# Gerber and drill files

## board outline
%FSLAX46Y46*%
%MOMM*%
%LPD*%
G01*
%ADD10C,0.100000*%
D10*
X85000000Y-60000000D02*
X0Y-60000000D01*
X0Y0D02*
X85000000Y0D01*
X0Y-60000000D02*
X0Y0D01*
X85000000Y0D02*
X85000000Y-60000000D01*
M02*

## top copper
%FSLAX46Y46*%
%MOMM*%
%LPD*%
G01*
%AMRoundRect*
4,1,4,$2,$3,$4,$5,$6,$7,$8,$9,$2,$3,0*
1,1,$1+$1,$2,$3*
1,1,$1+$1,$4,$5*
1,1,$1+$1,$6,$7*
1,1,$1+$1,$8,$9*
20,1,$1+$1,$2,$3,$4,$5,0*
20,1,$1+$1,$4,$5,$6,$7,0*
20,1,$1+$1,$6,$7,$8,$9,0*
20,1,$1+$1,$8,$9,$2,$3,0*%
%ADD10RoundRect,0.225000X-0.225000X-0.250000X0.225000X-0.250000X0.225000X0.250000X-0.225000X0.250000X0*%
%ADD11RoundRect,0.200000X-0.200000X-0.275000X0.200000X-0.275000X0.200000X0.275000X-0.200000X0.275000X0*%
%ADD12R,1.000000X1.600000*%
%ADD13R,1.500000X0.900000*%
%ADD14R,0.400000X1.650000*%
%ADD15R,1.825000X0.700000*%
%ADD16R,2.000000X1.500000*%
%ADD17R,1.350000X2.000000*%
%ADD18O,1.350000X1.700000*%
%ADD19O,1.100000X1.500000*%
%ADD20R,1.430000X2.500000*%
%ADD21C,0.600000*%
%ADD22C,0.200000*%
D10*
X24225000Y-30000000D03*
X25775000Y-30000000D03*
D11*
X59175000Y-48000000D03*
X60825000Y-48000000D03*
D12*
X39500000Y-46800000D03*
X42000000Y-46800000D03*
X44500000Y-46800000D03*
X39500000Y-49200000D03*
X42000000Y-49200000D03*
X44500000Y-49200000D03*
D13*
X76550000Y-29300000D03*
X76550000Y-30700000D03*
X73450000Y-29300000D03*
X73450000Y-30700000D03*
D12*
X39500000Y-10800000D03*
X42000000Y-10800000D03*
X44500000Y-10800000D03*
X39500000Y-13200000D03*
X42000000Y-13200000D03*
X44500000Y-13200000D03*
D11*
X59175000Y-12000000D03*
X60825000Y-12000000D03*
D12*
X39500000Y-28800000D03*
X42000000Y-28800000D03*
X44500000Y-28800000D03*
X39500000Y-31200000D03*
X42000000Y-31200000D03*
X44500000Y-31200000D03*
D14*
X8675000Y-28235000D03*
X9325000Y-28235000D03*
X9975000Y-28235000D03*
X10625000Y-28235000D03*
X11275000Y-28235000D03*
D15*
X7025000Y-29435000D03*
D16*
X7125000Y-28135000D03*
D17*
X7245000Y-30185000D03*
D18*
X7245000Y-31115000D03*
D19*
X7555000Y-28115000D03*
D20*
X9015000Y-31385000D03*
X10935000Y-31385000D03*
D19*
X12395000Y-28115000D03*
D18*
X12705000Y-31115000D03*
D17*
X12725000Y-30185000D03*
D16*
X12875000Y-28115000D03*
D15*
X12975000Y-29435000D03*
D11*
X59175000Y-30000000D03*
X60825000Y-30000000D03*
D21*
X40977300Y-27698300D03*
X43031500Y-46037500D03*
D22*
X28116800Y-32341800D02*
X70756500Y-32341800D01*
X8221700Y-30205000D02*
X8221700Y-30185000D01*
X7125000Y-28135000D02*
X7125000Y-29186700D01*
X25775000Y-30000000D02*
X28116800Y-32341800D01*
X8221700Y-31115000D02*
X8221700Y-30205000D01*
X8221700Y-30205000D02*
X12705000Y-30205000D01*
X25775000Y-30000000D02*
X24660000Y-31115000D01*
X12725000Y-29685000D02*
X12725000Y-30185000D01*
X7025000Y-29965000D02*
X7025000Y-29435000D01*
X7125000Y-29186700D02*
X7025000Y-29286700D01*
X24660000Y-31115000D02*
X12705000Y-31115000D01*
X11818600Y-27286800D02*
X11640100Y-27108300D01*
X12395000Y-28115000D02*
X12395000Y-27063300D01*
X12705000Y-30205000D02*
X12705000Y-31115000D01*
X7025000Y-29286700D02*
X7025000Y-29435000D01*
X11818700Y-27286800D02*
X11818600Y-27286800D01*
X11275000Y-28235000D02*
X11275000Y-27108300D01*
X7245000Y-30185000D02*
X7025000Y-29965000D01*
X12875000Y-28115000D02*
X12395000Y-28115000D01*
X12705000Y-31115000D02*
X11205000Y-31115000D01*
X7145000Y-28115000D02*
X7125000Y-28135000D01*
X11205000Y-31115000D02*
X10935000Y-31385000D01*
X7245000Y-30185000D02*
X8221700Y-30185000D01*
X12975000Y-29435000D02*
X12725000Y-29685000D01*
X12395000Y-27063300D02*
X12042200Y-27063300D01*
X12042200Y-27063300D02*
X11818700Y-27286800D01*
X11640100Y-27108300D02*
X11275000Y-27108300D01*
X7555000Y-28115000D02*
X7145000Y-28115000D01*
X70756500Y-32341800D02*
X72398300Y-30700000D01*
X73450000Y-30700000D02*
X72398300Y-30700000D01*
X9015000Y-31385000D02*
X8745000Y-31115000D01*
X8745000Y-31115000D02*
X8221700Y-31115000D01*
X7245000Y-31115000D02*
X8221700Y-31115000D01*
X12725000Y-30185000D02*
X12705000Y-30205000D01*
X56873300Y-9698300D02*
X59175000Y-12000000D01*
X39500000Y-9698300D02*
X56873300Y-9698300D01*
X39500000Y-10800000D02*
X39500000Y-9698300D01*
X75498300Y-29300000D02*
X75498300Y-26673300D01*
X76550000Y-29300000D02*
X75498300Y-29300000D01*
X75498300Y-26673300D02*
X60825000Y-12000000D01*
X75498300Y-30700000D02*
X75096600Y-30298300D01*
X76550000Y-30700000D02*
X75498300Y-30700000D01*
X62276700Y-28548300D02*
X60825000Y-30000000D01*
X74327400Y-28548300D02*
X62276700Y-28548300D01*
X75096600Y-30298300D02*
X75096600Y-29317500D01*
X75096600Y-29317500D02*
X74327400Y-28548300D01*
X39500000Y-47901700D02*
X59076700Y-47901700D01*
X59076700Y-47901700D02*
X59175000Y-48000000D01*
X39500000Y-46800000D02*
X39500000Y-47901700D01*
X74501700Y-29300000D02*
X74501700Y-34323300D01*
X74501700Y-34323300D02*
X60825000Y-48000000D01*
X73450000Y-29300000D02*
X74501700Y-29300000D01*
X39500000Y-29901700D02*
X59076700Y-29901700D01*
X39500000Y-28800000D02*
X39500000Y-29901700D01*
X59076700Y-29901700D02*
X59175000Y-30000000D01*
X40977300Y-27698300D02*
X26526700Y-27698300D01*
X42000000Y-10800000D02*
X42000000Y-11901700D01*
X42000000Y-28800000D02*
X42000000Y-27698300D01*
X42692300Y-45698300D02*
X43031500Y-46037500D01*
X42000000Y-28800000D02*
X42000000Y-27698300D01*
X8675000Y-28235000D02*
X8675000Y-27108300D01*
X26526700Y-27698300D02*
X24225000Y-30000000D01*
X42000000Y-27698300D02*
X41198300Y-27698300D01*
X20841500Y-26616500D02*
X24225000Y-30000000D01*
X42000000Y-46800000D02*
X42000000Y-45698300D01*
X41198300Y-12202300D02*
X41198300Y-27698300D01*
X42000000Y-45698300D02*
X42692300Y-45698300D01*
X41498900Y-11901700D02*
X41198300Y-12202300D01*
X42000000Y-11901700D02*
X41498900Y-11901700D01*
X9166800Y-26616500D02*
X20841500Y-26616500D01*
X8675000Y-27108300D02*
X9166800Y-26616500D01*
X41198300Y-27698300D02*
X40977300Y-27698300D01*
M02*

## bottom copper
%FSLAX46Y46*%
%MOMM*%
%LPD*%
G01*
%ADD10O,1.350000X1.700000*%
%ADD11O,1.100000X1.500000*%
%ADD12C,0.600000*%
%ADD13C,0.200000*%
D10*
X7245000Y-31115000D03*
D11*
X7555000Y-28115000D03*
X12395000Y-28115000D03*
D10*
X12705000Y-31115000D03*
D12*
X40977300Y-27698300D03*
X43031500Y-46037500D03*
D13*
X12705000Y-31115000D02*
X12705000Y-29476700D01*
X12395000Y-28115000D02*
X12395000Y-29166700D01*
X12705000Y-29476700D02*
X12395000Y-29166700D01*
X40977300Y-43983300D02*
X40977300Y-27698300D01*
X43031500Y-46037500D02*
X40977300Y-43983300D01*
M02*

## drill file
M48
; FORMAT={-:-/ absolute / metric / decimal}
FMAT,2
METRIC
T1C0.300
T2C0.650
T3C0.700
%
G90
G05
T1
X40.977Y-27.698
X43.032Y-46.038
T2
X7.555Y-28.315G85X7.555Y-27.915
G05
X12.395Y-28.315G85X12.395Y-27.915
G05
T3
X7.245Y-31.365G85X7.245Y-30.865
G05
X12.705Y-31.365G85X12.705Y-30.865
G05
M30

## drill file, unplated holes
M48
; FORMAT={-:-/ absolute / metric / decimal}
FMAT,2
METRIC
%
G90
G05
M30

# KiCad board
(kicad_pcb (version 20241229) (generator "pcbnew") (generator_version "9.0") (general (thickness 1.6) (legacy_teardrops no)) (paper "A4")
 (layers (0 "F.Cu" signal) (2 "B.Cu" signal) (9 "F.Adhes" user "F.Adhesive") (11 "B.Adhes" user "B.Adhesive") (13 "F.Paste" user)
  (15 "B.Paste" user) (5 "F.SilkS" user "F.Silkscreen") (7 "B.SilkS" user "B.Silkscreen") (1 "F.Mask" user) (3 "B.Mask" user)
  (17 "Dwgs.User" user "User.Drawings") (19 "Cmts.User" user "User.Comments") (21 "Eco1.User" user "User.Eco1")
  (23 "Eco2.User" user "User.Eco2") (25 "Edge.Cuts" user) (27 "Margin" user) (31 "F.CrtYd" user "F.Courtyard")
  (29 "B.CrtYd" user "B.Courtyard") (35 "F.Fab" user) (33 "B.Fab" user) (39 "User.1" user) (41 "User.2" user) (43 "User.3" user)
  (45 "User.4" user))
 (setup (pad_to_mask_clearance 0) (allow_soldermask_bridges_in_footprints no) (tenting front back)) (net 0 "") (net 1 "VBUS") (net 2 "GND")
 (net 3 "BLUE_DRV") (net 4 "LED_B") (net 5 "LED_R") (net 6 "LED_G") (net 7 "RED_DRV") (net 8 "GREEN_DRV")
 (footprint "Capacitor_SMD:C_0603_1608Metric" (layer "F.Cu") (at 25 30)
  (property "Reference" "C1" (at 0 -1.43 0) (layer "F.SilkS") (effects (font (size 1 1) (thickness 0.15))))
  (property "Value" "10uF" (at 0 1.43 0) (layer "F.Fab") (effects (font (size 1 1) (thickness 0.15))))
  (pad "1" smd roundrect (at -0.775 0) (size 0.9 0.95) (layers "F.Cu" "F.Mask" "F.Paste") (roundrect_rratio 0.25) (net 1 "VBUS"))
  (pad "2" smd roundrect (at 0.775 0) (size 0.9 0.95) (layers "F.Cu" "F.Mask" "F.Paste") (roundrect_rratio 0.25) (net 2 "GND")))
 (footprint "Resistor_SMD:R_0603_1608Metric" (layer "F.Cu") (at 60 48)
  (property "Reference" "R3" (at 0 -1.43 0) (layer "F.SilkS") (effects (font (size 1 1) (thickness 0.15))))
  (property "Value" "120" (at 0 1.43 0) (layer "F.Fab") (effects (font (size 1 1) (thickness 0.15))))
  (pad "1" smd roundrect (at -0.825 0) (size 0.8 0.95) (layers "F.Cu" "F.Mask" "F.Paste") (roundrect_rratio 0.25) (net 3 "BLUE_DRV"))
  (pad "2" smd roundrect (at 0.825 0) (size 0.8 0.95) (layers "F.Cu" "F.Mask" "F.Paste") (roundrect_rratio 0.25) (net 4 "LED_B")))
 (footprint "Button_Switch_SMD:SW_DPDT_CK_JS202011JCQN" (layer "F.Cu") (at 42 48)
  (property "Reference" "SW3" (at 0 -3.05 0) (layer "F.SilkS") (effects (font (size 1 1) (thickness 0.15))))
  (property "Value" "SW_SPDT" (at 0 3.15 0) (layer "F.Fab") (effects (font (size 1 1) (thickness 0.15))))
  (pad "1" smd rect (at -2.5 -1.2) (size 1 1.6) (layers "F.Cu" "F.Mask" "F.Paste") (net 3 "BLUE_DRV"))
  (pad "2" smd rect (at 0 -1.2) (size 1 1.6) (layers "F.Cu" "F.Mask" "F.Paste") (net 1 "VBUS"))
  (pad "3" smd rect (at 2.5 -1.2) (size 1 1.6) (layers "F.Cu" "F.Mask" "F.Paste"))
  (pad "4" smd rect (at -2.5 1.2) (size 1 1.6) (layers "F.Cu" "F.Mask" "F.Paste"))
  (pad "5" smd rect (at 0 1.2) (size 1 1.6) (layers "F.Cu" "F.Mask" "F.Paste"))
  (pad "6" smd rect (at 2.5 1.2) (size 1 1.6) (layers "F.Cu" "F.Mask" "F.Paste")))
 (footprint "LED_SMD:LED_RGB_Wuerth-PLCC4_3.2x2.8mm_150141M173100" (layer "F.Cu") (at 75 30)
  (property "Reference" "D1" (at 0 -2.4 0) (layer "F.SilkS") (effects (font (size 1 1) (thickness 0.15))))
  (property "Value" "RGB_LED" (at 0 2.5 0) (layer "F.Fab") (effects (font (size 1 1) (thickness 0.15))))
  (pad "1" smd rect (at 1.55 -0.7) (size 1.5 0.9) (layers "F.Cu" "F.Mask" "F.Paste") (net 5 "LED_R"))
  (pad "2" smd rect (at 1.55 0.7) (size 1.5 0.9) (layers "F.Cu" "F.Mask" "F.Paste") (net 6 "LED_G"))
  (pad "3" smd rect (at -1.55 -0.7) (size 1.5 0.9) (layers "F.Cu" "F.Mask" "F.Paste") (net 4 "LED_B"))
  (pad "4" smd rect (at -1.55 0.7) (size 1.5 0.9) (layers "F.Cu" "F.Mask" "F.Paste") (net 2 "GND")))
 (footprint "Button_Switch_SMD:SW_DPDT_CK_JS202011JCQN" (layer "F.Cu") (at 42 12)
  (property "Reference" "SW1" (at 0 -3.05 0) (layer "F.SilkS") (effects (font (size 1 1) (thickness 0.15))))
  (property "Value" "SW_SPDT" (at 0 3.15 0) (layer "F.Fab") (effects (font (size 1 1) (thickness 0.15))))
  (pad "1" smd rect (at -2.5 -1.2) (size 1 1.6) (layers "F.Cu" "F.Mask" "F.Paste") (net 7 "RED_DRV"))
  (pad "2" smd rect (at 0 -1.2) (size 1 1.6) (layers "F.Cu" "F.Mask" "F.Paste") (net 1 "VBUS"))
  (pad "3" smd rect (at 2.5 -1.2) (size 1 1.6) (layers "F.Cu" "F.Mask" "F.Paste"))
  (pad "4" smd rect (at -2.5 1.2) (size 1 1.6) (layers "F.Cu" "F.Mask" "F.Paste"))
  (pad "5" smd rect (at 0 1.2) (size 1 1.6) (layers "F.Cu" "F.Mask" "F.Paste"))
  (pad "6" smd rect (at 2.5 1.2) (size 1 1.6) (layers "F.Cu" "F.Mask" "F.Paste")))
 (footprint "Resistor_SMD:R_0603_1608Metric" (layer "F.Cu") (at 60 12)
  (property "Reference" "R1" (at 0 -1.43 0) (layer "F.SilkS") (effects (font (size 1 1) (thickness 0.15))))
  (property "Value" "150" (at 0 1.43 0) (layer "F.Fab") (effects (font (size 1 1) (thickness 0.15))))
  (pad "1" smd roundrect (at -0.825 0) (size 0.8 0.95) (layers "F.Cu" "F.Mask" "F.Paste") (roundrect_rratio 0.25) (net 7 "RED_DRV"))
  (pad "2" smd roundrect (at 0.825 0) (size 0.8 0.95) (layers "F.Cu" "F.Mask" "F.Paste") (roundrect_rratio 0.25) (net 5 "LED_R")))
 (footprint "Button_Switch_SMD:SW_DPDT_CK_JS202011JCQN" (layer "F.Cu") (at 42 30)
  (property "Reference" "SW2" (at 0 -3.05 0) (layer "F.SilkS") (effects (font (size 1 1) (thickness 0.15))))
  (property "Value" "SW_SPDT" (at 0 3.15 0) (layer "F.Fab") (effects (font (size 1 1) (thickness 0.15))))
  (pad "1" smd rect (at -2.5 -1.2) (size 1 1.6) (layers "F.Cu" "F.Mask" "F.Paste") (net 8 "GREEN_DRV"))
  (pad "2" smd rect (at 0 -1.2) (size 1 1.6) (layers "F.Cu" "F.Mask" "F.Paste") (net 1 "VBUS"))
  (pad "3" smd rect (at 2.5 -1.2) (size 1 1.6) (layers "F.Cu" "F.Mask" "F.Paste"))
  (pad "4" smd rect (at -2.5 1.2) (size 1 1.6) (layers "F.Cu" "F.Mask" "F.Paste"))
  (pad "5" smd rect (at 0 1.2) (size 1 1.6) (layers "F.Cu" "F.Mask" "F.Paste"))
  (pad "6" smd rect (at 2.5 1.2) (size 1 1.6) (layers "F.Cu" "F.Mask" "F.Paste")))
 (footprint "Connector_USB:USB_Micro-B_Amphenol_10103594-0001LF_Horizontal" (layer "F.Cu") (at 10 30)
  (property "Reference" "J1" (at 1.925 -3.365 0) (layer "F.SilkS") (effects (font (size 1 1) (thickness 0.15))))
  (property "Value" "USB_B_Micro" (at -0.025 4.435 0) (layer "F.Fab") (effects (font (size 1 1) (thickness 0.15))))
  (pad "1" smd rect (at -1.325 -1.765 90) (size 1.65 0.4) (layers "F.Cu" "F.Mask" "F.Paste") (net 1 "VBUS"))
  (pad "2" smd rect (at -0.675 -1.765 90) (size 1.65 0.4) (layers "F.Cu" "F.Mask" "F.Paste"))
  (pad "3" smd rect (at -0.025 -1.765 90) (size 1.65 0.4) (layers "F.Cu" "F.Mask" "F.Paste"))
  (pad "4" smd rect (at 0.625 -1.765 90) (size 1.65 0.4) (layers "F.Cu" "F.Mask" "F.Paste"))
  (pad "5" smd rect (at 1.275 -1.765 90) (size 1.65 0.4) (layers "F.Cu" "F.Mask" "F.Paste") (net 2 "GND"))
  (pad "6" smd rect (at -2.975 -0.565) (size 1.825 0.7) (layers "F.Cu" "F.Mask" "F.Paste") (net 2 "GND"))
  (pad "6" smd rect (at -2.875 -1.865) (size 2 1.5) (layers "F.Cu" "F.Mask" "F.Paste") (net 2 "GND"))
  (pad "6" smd rect (at -2.755 0.185) (size 1.35 2) (layers "F.Cu" "F.Mask" "F.Paste") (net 2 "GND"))
  (pad "6" thru_hole oval (at -2.755 1.115 90) (size 1.7 1.35) (drill oval 1.2 0.7) (layers "*.Cu" "*.Mask") (remove_unused_layers no)
   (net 2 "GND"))
  (pad "6" thru_hole oval (at -2.445 -1.885 90) (size 1.5 1.1) (drill oval 1.05 0.65) (layers "*.Cu" "*.Mask") (remove_unused_layers no)
   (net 2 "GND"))
  (pad "6" smd rect (at -0.985 1.385 90) (size 2.5 1.43) (layers "F.Cu" "F.Mask" "F.Paste") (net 2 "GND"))
  (pad "6" smd rect (at 0.935 1.385 90) (size 2.5 1.43) (layers "F.Cu" "F.Mask" "F.Paste") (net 2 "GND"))
  (pad "6" thru_hole oval (at 2.395 -1.885 90) (size 1.5 1.1) (drill oval 1.05 0.65) (layers "*.Cu" "*.Mask") (remove_unused_layers no)
   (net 2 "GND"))
  (pad "6" thru_hole oval (at 2.705 1.115 90) (size 1.7 1.35) (drill oval 1.2 0.7) (layers "*.Cu" "*.Mask") (remove_unused_layers no)
   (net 2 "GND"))
  (pad "6" smd rect (at 2.725 0.185) (size 1.35 2) (layers "F.Cu" "F.Mask" "F.Paste") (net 2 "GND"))
  (pad "6" smd rect (at 2.875 -1.885) (size 2 1.5) (layers "F.Cu" "F.Mask" "F.Paste") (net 2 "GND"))
  (pad "6" smd rect (at 2.975 -0.565) (size 1.825 0.7) (layers "F.Cu" "F.Mask" "F.Paste") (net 2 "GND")))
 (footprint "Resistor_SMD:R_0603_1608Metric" (layer "F.Cu") (at 60 30)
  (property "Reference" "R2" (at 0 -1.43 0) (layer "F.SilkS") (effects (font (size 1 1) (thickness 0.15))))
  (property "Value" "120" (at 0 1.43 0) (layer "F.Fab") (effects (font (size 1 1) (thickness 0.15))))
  (pad "1" smd roundrect (at -0.825 0) (size 0.8 0.95) (layers "F.Cu" "F.Mask" "F.Paste") (roundrect_rratio 0.25) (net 8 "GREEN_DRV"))
  (pad "2" smd roundrect (at 0.825 0) (size 0.8 0.95) (layers "F.Cu" "F.Mask" "F.Paste") (roundrect_rratio 0.25) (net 6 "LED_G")))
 (gr_line (start 85 60) (end 0 60) (stroke (width 0) (type default)) (layer "Edge.Cuts"))
 (gr_line (start 0 0) (end 85 0) (stroke (width 0) (type default)) (layer "Edge.Cuts"))
 (gr_line (start 0 60) (end 0 0) (stroke (width 0) (type default)) (layer "Edge.Cuts"))
 (gr_line (start 85 0) (end 85 60) (stroke (width 0) (type default)) (layer "Edge.Cuts"))
 (segment (start 28.1168 32.3418) (end 70.7565 32.3418) (width 0.2) (layer "F.Cu") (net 2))
 (segment (start 8.2217 30.205) (end 8.2217 30.185) (width 0.2) (layer "F.Cu") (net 2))
 (segment (start 7.125 28.135) (end 7.125 29.1867) (width 0.2) (layer "F.Cu") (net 2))
 (segment (start 25.775 30) (end 28.1168 32.3418) (width 0.2) (layer "F.Cu") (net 2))
 (segment (start 8.2217 31.115) (end 8.2217 30.205) (width 0.2) (layer "F.Cu") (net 2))
 (segment (start 8.2217 30.205) (end 12.705 30.205) (width 0.2) (layer "F.Cu") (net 2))
 (segment (start 25.775 30) (end 24.66 31.115) (width 0.2) (layer "F.Cu") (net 2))
 (segment (start 12.725 29.685) (end 12.725 30.185) (width 0.2) (layer "F.Cu") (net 2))
 (segment (start 7.025 29.965) (end 7.025 29.435) (width 0.2) (layer "F.Cu") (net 2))
 (segment (start 7.125 29.1867) (end 7.025 29.2867) (width 0.2) (layer "F.Cu") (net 2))
 (segment (start 24.66 31.115) (end 12.705 31.115) (width 0.2) (layer "F.Cu") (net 2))
 (segment (start 11.8186 27.2868) (end 11.6401 27.1083) (width 0.2) (layer "F.Cu") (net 2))
 (segment (start 12.395 28.115) (end 12.395 27.0633) (width 0.2) (layer "F.Cu") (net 2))
 (segment (start 12.705 30.205) (end 12.705 31.115) (width 0.2) (layer "F.Cu") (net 2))
 (segment (start 7.025 29.2867) (end 7.025 29.435) (width 0.2) (layer "F.Cu") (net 2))
 (segment (start 11.8187 27.2868) (end 11.8186 27.2868) (width 0.2) (layer "F.Cu") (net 2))
 (segment (start 11.275 28.235) (end 11.275 27.1083) (width 0.2) (layer "F.Cu") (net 2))
 (segment (start 7.245 30.185) (end 7.025 29.965) (width 0.2) (layer "F.Cu") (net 2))
 (segment (start 12.875 28.115) (end 12.395 28.115) (width 0.2) (layer "F.Cu") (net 2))
 (segment (start 12.705 31.115) (end 11.205 31.115) (width 0.2) (layer "F.Cu") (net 2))
 (segment (start 7.145 28.115) (end 7.125 28.135) (width 0.2) (layer "F.Cu") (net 2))
 (segment (start 11.205 31.115) (end 10.935 31.385) (width 0.2) (layer "F.Cu") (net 2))
 (segment (start 7.245 30.185) (end 8.2217 30.185) (width 0.2) (layer "F.Cu") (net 2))
 (segment (start 12.975 29.435) (end 12.725 29.685) (width 0.2) (layer "F.Cu") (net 2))
 (segment (start 12.395 27.0633) (end 12.0422 27.0633) (width 0.2) (layer "F.Cu") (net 2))
 (segment (start 12.0422 27.0633) (end 11.8187 27.2868) (width 0.2) (layer "F.Cu") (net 2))
 (segment (start 11.6401 27.1083) (end 11.275 27.1083) (width 0.2) (layer "F.Cu") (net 2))
 (segment (start 7.555 28.115) (end 7.145 28.115) (width 0.2) (layer "F.Cu") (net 2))
 (segment (start 70.7565 32.3418) (end 72.3983 30.7) (width 0.2) (layer "F.Cu") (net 2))
 (segment (start 73.45 30.7) (end 72.3983 30.7) (width 0.2) (layer "F.Cu") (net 2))
 (segment (start 9.015 31.385) (end 8.745 31.115) (width 0.2) (layer "F.Cu") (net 2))
 (segment (start 8.745 31.115) (end 8.2217 31.115) (width 0.2) (layer "F.Cu") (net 2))
 (segment (start 7.245 31.115) (end 8.2217 31.115) (width 0.2) (layer "F.Cu") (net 2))
 (segment (start 12.725 30.185) (end 12.705 30.205) (width 0.2) (layer "F.Cu") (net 2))
 (segment (start 12.705 31.115) (end 12.705 29.4767) (width 0.2) (layer "B.Cu") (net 2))
 (segment (start 12.395 28.115) (end 12.395 29.1667) (width 0.2) (layer "B.Cu") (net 2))
 (segment (start 12.705 29.4767) (end 12.395 29.1667) (width 0.2) (layer "B.Cu") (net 2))
 (segment (start 56.8733 9.6983) (end 59.175 12) (width 0.2) (layer "F.Cu") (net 7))
 (segment (start 39.5 9.6983) (end 56.8733 9.6983) (width 0.2) (layer "F.Cu") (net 7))
 (segment (start 39.5 10.8) (end 39.5 9.6983) (width 0.2) (layer "F.Cu") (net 7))
 (segment (start 75.4983 29.3) (end 75.4983 26.6733) (width 0.2) (layer "F.Cu") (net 5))
 (segment (start 76.55 29.3) (end 75.4983 29.3) (width 0.2) (layer "F.Cu") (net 5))
 (segment (start 75.4983 26.6733) (end 60.825 12) (width 0.2) (layer "F.Cu") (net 5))
 (segment (start 75.4983 30.7) (end 75.0966 30.2983) (width 0.2) (layer "F.Cu") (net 6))
 (segment (start 76.55 30.7) (end 75.4983 30.7) (width 0.2) (layer "F.Cu") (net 6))
 (segment (start 62.2767 28.5483) (end 60.825 30) (width 0.2) (layer "F.Cu") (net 6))
 (segment (start 74.3274 28.5483) (end 62.2767 28.5483) (width 0.2) (layer "F.Cu") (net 6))
 (segment (start 75.0966 30.2983) (end 75.0966 29.3175) (width 0.2) (layer "F.Cu") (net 6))
 (segment (start 75.0966 29.3175) (end 74.3274 28.5483) (width 0.2) (layer "F.Cu") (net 6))
 (segment (start 39.5 47.9017) (end 59.0767 47.9017) (width 0.2) (layer "F.Cu") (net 3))
 (segment (start 59.0767 47.9017) (end 59.175 48) (width 0.2) (layer "F.Cu") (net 3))
 (segment (start 39.5 46.8) (end 39.5 47.9017) (width 0.2) (layer "F.Cu") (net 3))
 (segment (start 74.5017 29.3) (end 74.5017 34.3233) (width 0.2) (layer "F.Cu") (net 4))
 (segment (start 74.5017 34.3233) (end 60.825 48) (width 0.2) (layer "F.Cu") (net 4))
 (segment (start 73.45 29.3) (end 74.5017 29.3) (width 0.2) (layer "F.Cu") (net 4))
 (segment (start 39.5 29.9017) (end 59.0767 29.9017) (width 0.2) (layer "F.Cu") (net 8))
 (segment (start 39.5 28.8) (end 39.5 29.9017) (width 0.2) (layer "F.Cu") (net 8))
 (segment (start 59.0767 29.9017) (end 59.175 30) (width 0.2) (layer "F.Cu") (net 8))
 (segment (start 40.9773 27.6983) (end 26.5267 27.6983) (width 0.2) (layer "F.Cu") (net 1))
 (segment (start 42 10.8) (end 42 11.9017) (width 0.2) (layer "F.Cu") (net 1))
 (segment (start 42 28.8) (end 42 27.6983) (width 0.2) (layer "F.Cu") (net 1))
 (segment (start 42.6923 45.6983) (end 43.0315 46.0375) (width 0.2) (layer "F.Cu") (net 1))
 (segment (start 42 28.8) (end 42 27.6983) (width 0.2) (layer "F.Cu") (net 1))
 (segment (start 8.675 28.235) (end 8.675 27.1083) (width 0.2) (layer "F.Cu") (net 1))
 (segment (start 26.5267 27.6983) (end 24.225 30) (width 0.2) (layer "F.Cu") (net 1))
 (segment (start 42 27.6983) (end 41.1983 27.6983) (width 0.2) (layer "F.Cu") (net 1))
 (segment (start 20.8415 26.6165) (end 24.225 30) (width 0.2) (layer "F.Cu") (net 1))
 (segment (start 42 46.8) (end 42 45.6983) (width 0.2) (layer "F.Cu") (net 1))
 (segment (start 41.1983 12.2023) (end 41.1983 27.6983) (width 0.2) (layer "F.Cu") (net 1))
 (segment (start 42 45.6983) (end 42.6923 45.6983) (width 0.2) (layer "F.Cu") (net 1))
 (segment (start 41.4989 11.9017) (end 41.1983 12.2023) (width 0.2) (layer "F.Cu") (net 1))
 (segment (start 42 11.9017) (end 41.4989 11.9017) (width 0.2) (layer "F.Cu") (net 1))
 (segment (start 9.1668 26.6165) (end 20.8415 26.6165) (width 0.2) (layer "F.Cu") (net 1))
 (segment (start 8.675 27.1083) (end 9.1668 26.6165) (width 0.2) (layer "F.Cu") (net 1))
 (segment (start 41.1983 27.6983) (end 40.9773 27.6983) (width 0.2) (layer "F.Cu") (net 1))
 (via (at 40.9773 27.6983) (size 0.6) (drill 0.3) (layers "F.Cu" "B.Cu") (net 1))
 (via (at 43.0315 46.0375) (size 0.6) (drill 0.3) (layers "F.Cu" "B.Cu") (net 1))
 (segment (start 40.9773 43.9833) (end 40.9773 27.6983) (width 0.2) (layer "B.Cu") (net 1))
 (segment (start 43.0315 46.0375) (end 40.9773 43.9833) (width 0.2) (layer "B.Cu") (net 1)))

